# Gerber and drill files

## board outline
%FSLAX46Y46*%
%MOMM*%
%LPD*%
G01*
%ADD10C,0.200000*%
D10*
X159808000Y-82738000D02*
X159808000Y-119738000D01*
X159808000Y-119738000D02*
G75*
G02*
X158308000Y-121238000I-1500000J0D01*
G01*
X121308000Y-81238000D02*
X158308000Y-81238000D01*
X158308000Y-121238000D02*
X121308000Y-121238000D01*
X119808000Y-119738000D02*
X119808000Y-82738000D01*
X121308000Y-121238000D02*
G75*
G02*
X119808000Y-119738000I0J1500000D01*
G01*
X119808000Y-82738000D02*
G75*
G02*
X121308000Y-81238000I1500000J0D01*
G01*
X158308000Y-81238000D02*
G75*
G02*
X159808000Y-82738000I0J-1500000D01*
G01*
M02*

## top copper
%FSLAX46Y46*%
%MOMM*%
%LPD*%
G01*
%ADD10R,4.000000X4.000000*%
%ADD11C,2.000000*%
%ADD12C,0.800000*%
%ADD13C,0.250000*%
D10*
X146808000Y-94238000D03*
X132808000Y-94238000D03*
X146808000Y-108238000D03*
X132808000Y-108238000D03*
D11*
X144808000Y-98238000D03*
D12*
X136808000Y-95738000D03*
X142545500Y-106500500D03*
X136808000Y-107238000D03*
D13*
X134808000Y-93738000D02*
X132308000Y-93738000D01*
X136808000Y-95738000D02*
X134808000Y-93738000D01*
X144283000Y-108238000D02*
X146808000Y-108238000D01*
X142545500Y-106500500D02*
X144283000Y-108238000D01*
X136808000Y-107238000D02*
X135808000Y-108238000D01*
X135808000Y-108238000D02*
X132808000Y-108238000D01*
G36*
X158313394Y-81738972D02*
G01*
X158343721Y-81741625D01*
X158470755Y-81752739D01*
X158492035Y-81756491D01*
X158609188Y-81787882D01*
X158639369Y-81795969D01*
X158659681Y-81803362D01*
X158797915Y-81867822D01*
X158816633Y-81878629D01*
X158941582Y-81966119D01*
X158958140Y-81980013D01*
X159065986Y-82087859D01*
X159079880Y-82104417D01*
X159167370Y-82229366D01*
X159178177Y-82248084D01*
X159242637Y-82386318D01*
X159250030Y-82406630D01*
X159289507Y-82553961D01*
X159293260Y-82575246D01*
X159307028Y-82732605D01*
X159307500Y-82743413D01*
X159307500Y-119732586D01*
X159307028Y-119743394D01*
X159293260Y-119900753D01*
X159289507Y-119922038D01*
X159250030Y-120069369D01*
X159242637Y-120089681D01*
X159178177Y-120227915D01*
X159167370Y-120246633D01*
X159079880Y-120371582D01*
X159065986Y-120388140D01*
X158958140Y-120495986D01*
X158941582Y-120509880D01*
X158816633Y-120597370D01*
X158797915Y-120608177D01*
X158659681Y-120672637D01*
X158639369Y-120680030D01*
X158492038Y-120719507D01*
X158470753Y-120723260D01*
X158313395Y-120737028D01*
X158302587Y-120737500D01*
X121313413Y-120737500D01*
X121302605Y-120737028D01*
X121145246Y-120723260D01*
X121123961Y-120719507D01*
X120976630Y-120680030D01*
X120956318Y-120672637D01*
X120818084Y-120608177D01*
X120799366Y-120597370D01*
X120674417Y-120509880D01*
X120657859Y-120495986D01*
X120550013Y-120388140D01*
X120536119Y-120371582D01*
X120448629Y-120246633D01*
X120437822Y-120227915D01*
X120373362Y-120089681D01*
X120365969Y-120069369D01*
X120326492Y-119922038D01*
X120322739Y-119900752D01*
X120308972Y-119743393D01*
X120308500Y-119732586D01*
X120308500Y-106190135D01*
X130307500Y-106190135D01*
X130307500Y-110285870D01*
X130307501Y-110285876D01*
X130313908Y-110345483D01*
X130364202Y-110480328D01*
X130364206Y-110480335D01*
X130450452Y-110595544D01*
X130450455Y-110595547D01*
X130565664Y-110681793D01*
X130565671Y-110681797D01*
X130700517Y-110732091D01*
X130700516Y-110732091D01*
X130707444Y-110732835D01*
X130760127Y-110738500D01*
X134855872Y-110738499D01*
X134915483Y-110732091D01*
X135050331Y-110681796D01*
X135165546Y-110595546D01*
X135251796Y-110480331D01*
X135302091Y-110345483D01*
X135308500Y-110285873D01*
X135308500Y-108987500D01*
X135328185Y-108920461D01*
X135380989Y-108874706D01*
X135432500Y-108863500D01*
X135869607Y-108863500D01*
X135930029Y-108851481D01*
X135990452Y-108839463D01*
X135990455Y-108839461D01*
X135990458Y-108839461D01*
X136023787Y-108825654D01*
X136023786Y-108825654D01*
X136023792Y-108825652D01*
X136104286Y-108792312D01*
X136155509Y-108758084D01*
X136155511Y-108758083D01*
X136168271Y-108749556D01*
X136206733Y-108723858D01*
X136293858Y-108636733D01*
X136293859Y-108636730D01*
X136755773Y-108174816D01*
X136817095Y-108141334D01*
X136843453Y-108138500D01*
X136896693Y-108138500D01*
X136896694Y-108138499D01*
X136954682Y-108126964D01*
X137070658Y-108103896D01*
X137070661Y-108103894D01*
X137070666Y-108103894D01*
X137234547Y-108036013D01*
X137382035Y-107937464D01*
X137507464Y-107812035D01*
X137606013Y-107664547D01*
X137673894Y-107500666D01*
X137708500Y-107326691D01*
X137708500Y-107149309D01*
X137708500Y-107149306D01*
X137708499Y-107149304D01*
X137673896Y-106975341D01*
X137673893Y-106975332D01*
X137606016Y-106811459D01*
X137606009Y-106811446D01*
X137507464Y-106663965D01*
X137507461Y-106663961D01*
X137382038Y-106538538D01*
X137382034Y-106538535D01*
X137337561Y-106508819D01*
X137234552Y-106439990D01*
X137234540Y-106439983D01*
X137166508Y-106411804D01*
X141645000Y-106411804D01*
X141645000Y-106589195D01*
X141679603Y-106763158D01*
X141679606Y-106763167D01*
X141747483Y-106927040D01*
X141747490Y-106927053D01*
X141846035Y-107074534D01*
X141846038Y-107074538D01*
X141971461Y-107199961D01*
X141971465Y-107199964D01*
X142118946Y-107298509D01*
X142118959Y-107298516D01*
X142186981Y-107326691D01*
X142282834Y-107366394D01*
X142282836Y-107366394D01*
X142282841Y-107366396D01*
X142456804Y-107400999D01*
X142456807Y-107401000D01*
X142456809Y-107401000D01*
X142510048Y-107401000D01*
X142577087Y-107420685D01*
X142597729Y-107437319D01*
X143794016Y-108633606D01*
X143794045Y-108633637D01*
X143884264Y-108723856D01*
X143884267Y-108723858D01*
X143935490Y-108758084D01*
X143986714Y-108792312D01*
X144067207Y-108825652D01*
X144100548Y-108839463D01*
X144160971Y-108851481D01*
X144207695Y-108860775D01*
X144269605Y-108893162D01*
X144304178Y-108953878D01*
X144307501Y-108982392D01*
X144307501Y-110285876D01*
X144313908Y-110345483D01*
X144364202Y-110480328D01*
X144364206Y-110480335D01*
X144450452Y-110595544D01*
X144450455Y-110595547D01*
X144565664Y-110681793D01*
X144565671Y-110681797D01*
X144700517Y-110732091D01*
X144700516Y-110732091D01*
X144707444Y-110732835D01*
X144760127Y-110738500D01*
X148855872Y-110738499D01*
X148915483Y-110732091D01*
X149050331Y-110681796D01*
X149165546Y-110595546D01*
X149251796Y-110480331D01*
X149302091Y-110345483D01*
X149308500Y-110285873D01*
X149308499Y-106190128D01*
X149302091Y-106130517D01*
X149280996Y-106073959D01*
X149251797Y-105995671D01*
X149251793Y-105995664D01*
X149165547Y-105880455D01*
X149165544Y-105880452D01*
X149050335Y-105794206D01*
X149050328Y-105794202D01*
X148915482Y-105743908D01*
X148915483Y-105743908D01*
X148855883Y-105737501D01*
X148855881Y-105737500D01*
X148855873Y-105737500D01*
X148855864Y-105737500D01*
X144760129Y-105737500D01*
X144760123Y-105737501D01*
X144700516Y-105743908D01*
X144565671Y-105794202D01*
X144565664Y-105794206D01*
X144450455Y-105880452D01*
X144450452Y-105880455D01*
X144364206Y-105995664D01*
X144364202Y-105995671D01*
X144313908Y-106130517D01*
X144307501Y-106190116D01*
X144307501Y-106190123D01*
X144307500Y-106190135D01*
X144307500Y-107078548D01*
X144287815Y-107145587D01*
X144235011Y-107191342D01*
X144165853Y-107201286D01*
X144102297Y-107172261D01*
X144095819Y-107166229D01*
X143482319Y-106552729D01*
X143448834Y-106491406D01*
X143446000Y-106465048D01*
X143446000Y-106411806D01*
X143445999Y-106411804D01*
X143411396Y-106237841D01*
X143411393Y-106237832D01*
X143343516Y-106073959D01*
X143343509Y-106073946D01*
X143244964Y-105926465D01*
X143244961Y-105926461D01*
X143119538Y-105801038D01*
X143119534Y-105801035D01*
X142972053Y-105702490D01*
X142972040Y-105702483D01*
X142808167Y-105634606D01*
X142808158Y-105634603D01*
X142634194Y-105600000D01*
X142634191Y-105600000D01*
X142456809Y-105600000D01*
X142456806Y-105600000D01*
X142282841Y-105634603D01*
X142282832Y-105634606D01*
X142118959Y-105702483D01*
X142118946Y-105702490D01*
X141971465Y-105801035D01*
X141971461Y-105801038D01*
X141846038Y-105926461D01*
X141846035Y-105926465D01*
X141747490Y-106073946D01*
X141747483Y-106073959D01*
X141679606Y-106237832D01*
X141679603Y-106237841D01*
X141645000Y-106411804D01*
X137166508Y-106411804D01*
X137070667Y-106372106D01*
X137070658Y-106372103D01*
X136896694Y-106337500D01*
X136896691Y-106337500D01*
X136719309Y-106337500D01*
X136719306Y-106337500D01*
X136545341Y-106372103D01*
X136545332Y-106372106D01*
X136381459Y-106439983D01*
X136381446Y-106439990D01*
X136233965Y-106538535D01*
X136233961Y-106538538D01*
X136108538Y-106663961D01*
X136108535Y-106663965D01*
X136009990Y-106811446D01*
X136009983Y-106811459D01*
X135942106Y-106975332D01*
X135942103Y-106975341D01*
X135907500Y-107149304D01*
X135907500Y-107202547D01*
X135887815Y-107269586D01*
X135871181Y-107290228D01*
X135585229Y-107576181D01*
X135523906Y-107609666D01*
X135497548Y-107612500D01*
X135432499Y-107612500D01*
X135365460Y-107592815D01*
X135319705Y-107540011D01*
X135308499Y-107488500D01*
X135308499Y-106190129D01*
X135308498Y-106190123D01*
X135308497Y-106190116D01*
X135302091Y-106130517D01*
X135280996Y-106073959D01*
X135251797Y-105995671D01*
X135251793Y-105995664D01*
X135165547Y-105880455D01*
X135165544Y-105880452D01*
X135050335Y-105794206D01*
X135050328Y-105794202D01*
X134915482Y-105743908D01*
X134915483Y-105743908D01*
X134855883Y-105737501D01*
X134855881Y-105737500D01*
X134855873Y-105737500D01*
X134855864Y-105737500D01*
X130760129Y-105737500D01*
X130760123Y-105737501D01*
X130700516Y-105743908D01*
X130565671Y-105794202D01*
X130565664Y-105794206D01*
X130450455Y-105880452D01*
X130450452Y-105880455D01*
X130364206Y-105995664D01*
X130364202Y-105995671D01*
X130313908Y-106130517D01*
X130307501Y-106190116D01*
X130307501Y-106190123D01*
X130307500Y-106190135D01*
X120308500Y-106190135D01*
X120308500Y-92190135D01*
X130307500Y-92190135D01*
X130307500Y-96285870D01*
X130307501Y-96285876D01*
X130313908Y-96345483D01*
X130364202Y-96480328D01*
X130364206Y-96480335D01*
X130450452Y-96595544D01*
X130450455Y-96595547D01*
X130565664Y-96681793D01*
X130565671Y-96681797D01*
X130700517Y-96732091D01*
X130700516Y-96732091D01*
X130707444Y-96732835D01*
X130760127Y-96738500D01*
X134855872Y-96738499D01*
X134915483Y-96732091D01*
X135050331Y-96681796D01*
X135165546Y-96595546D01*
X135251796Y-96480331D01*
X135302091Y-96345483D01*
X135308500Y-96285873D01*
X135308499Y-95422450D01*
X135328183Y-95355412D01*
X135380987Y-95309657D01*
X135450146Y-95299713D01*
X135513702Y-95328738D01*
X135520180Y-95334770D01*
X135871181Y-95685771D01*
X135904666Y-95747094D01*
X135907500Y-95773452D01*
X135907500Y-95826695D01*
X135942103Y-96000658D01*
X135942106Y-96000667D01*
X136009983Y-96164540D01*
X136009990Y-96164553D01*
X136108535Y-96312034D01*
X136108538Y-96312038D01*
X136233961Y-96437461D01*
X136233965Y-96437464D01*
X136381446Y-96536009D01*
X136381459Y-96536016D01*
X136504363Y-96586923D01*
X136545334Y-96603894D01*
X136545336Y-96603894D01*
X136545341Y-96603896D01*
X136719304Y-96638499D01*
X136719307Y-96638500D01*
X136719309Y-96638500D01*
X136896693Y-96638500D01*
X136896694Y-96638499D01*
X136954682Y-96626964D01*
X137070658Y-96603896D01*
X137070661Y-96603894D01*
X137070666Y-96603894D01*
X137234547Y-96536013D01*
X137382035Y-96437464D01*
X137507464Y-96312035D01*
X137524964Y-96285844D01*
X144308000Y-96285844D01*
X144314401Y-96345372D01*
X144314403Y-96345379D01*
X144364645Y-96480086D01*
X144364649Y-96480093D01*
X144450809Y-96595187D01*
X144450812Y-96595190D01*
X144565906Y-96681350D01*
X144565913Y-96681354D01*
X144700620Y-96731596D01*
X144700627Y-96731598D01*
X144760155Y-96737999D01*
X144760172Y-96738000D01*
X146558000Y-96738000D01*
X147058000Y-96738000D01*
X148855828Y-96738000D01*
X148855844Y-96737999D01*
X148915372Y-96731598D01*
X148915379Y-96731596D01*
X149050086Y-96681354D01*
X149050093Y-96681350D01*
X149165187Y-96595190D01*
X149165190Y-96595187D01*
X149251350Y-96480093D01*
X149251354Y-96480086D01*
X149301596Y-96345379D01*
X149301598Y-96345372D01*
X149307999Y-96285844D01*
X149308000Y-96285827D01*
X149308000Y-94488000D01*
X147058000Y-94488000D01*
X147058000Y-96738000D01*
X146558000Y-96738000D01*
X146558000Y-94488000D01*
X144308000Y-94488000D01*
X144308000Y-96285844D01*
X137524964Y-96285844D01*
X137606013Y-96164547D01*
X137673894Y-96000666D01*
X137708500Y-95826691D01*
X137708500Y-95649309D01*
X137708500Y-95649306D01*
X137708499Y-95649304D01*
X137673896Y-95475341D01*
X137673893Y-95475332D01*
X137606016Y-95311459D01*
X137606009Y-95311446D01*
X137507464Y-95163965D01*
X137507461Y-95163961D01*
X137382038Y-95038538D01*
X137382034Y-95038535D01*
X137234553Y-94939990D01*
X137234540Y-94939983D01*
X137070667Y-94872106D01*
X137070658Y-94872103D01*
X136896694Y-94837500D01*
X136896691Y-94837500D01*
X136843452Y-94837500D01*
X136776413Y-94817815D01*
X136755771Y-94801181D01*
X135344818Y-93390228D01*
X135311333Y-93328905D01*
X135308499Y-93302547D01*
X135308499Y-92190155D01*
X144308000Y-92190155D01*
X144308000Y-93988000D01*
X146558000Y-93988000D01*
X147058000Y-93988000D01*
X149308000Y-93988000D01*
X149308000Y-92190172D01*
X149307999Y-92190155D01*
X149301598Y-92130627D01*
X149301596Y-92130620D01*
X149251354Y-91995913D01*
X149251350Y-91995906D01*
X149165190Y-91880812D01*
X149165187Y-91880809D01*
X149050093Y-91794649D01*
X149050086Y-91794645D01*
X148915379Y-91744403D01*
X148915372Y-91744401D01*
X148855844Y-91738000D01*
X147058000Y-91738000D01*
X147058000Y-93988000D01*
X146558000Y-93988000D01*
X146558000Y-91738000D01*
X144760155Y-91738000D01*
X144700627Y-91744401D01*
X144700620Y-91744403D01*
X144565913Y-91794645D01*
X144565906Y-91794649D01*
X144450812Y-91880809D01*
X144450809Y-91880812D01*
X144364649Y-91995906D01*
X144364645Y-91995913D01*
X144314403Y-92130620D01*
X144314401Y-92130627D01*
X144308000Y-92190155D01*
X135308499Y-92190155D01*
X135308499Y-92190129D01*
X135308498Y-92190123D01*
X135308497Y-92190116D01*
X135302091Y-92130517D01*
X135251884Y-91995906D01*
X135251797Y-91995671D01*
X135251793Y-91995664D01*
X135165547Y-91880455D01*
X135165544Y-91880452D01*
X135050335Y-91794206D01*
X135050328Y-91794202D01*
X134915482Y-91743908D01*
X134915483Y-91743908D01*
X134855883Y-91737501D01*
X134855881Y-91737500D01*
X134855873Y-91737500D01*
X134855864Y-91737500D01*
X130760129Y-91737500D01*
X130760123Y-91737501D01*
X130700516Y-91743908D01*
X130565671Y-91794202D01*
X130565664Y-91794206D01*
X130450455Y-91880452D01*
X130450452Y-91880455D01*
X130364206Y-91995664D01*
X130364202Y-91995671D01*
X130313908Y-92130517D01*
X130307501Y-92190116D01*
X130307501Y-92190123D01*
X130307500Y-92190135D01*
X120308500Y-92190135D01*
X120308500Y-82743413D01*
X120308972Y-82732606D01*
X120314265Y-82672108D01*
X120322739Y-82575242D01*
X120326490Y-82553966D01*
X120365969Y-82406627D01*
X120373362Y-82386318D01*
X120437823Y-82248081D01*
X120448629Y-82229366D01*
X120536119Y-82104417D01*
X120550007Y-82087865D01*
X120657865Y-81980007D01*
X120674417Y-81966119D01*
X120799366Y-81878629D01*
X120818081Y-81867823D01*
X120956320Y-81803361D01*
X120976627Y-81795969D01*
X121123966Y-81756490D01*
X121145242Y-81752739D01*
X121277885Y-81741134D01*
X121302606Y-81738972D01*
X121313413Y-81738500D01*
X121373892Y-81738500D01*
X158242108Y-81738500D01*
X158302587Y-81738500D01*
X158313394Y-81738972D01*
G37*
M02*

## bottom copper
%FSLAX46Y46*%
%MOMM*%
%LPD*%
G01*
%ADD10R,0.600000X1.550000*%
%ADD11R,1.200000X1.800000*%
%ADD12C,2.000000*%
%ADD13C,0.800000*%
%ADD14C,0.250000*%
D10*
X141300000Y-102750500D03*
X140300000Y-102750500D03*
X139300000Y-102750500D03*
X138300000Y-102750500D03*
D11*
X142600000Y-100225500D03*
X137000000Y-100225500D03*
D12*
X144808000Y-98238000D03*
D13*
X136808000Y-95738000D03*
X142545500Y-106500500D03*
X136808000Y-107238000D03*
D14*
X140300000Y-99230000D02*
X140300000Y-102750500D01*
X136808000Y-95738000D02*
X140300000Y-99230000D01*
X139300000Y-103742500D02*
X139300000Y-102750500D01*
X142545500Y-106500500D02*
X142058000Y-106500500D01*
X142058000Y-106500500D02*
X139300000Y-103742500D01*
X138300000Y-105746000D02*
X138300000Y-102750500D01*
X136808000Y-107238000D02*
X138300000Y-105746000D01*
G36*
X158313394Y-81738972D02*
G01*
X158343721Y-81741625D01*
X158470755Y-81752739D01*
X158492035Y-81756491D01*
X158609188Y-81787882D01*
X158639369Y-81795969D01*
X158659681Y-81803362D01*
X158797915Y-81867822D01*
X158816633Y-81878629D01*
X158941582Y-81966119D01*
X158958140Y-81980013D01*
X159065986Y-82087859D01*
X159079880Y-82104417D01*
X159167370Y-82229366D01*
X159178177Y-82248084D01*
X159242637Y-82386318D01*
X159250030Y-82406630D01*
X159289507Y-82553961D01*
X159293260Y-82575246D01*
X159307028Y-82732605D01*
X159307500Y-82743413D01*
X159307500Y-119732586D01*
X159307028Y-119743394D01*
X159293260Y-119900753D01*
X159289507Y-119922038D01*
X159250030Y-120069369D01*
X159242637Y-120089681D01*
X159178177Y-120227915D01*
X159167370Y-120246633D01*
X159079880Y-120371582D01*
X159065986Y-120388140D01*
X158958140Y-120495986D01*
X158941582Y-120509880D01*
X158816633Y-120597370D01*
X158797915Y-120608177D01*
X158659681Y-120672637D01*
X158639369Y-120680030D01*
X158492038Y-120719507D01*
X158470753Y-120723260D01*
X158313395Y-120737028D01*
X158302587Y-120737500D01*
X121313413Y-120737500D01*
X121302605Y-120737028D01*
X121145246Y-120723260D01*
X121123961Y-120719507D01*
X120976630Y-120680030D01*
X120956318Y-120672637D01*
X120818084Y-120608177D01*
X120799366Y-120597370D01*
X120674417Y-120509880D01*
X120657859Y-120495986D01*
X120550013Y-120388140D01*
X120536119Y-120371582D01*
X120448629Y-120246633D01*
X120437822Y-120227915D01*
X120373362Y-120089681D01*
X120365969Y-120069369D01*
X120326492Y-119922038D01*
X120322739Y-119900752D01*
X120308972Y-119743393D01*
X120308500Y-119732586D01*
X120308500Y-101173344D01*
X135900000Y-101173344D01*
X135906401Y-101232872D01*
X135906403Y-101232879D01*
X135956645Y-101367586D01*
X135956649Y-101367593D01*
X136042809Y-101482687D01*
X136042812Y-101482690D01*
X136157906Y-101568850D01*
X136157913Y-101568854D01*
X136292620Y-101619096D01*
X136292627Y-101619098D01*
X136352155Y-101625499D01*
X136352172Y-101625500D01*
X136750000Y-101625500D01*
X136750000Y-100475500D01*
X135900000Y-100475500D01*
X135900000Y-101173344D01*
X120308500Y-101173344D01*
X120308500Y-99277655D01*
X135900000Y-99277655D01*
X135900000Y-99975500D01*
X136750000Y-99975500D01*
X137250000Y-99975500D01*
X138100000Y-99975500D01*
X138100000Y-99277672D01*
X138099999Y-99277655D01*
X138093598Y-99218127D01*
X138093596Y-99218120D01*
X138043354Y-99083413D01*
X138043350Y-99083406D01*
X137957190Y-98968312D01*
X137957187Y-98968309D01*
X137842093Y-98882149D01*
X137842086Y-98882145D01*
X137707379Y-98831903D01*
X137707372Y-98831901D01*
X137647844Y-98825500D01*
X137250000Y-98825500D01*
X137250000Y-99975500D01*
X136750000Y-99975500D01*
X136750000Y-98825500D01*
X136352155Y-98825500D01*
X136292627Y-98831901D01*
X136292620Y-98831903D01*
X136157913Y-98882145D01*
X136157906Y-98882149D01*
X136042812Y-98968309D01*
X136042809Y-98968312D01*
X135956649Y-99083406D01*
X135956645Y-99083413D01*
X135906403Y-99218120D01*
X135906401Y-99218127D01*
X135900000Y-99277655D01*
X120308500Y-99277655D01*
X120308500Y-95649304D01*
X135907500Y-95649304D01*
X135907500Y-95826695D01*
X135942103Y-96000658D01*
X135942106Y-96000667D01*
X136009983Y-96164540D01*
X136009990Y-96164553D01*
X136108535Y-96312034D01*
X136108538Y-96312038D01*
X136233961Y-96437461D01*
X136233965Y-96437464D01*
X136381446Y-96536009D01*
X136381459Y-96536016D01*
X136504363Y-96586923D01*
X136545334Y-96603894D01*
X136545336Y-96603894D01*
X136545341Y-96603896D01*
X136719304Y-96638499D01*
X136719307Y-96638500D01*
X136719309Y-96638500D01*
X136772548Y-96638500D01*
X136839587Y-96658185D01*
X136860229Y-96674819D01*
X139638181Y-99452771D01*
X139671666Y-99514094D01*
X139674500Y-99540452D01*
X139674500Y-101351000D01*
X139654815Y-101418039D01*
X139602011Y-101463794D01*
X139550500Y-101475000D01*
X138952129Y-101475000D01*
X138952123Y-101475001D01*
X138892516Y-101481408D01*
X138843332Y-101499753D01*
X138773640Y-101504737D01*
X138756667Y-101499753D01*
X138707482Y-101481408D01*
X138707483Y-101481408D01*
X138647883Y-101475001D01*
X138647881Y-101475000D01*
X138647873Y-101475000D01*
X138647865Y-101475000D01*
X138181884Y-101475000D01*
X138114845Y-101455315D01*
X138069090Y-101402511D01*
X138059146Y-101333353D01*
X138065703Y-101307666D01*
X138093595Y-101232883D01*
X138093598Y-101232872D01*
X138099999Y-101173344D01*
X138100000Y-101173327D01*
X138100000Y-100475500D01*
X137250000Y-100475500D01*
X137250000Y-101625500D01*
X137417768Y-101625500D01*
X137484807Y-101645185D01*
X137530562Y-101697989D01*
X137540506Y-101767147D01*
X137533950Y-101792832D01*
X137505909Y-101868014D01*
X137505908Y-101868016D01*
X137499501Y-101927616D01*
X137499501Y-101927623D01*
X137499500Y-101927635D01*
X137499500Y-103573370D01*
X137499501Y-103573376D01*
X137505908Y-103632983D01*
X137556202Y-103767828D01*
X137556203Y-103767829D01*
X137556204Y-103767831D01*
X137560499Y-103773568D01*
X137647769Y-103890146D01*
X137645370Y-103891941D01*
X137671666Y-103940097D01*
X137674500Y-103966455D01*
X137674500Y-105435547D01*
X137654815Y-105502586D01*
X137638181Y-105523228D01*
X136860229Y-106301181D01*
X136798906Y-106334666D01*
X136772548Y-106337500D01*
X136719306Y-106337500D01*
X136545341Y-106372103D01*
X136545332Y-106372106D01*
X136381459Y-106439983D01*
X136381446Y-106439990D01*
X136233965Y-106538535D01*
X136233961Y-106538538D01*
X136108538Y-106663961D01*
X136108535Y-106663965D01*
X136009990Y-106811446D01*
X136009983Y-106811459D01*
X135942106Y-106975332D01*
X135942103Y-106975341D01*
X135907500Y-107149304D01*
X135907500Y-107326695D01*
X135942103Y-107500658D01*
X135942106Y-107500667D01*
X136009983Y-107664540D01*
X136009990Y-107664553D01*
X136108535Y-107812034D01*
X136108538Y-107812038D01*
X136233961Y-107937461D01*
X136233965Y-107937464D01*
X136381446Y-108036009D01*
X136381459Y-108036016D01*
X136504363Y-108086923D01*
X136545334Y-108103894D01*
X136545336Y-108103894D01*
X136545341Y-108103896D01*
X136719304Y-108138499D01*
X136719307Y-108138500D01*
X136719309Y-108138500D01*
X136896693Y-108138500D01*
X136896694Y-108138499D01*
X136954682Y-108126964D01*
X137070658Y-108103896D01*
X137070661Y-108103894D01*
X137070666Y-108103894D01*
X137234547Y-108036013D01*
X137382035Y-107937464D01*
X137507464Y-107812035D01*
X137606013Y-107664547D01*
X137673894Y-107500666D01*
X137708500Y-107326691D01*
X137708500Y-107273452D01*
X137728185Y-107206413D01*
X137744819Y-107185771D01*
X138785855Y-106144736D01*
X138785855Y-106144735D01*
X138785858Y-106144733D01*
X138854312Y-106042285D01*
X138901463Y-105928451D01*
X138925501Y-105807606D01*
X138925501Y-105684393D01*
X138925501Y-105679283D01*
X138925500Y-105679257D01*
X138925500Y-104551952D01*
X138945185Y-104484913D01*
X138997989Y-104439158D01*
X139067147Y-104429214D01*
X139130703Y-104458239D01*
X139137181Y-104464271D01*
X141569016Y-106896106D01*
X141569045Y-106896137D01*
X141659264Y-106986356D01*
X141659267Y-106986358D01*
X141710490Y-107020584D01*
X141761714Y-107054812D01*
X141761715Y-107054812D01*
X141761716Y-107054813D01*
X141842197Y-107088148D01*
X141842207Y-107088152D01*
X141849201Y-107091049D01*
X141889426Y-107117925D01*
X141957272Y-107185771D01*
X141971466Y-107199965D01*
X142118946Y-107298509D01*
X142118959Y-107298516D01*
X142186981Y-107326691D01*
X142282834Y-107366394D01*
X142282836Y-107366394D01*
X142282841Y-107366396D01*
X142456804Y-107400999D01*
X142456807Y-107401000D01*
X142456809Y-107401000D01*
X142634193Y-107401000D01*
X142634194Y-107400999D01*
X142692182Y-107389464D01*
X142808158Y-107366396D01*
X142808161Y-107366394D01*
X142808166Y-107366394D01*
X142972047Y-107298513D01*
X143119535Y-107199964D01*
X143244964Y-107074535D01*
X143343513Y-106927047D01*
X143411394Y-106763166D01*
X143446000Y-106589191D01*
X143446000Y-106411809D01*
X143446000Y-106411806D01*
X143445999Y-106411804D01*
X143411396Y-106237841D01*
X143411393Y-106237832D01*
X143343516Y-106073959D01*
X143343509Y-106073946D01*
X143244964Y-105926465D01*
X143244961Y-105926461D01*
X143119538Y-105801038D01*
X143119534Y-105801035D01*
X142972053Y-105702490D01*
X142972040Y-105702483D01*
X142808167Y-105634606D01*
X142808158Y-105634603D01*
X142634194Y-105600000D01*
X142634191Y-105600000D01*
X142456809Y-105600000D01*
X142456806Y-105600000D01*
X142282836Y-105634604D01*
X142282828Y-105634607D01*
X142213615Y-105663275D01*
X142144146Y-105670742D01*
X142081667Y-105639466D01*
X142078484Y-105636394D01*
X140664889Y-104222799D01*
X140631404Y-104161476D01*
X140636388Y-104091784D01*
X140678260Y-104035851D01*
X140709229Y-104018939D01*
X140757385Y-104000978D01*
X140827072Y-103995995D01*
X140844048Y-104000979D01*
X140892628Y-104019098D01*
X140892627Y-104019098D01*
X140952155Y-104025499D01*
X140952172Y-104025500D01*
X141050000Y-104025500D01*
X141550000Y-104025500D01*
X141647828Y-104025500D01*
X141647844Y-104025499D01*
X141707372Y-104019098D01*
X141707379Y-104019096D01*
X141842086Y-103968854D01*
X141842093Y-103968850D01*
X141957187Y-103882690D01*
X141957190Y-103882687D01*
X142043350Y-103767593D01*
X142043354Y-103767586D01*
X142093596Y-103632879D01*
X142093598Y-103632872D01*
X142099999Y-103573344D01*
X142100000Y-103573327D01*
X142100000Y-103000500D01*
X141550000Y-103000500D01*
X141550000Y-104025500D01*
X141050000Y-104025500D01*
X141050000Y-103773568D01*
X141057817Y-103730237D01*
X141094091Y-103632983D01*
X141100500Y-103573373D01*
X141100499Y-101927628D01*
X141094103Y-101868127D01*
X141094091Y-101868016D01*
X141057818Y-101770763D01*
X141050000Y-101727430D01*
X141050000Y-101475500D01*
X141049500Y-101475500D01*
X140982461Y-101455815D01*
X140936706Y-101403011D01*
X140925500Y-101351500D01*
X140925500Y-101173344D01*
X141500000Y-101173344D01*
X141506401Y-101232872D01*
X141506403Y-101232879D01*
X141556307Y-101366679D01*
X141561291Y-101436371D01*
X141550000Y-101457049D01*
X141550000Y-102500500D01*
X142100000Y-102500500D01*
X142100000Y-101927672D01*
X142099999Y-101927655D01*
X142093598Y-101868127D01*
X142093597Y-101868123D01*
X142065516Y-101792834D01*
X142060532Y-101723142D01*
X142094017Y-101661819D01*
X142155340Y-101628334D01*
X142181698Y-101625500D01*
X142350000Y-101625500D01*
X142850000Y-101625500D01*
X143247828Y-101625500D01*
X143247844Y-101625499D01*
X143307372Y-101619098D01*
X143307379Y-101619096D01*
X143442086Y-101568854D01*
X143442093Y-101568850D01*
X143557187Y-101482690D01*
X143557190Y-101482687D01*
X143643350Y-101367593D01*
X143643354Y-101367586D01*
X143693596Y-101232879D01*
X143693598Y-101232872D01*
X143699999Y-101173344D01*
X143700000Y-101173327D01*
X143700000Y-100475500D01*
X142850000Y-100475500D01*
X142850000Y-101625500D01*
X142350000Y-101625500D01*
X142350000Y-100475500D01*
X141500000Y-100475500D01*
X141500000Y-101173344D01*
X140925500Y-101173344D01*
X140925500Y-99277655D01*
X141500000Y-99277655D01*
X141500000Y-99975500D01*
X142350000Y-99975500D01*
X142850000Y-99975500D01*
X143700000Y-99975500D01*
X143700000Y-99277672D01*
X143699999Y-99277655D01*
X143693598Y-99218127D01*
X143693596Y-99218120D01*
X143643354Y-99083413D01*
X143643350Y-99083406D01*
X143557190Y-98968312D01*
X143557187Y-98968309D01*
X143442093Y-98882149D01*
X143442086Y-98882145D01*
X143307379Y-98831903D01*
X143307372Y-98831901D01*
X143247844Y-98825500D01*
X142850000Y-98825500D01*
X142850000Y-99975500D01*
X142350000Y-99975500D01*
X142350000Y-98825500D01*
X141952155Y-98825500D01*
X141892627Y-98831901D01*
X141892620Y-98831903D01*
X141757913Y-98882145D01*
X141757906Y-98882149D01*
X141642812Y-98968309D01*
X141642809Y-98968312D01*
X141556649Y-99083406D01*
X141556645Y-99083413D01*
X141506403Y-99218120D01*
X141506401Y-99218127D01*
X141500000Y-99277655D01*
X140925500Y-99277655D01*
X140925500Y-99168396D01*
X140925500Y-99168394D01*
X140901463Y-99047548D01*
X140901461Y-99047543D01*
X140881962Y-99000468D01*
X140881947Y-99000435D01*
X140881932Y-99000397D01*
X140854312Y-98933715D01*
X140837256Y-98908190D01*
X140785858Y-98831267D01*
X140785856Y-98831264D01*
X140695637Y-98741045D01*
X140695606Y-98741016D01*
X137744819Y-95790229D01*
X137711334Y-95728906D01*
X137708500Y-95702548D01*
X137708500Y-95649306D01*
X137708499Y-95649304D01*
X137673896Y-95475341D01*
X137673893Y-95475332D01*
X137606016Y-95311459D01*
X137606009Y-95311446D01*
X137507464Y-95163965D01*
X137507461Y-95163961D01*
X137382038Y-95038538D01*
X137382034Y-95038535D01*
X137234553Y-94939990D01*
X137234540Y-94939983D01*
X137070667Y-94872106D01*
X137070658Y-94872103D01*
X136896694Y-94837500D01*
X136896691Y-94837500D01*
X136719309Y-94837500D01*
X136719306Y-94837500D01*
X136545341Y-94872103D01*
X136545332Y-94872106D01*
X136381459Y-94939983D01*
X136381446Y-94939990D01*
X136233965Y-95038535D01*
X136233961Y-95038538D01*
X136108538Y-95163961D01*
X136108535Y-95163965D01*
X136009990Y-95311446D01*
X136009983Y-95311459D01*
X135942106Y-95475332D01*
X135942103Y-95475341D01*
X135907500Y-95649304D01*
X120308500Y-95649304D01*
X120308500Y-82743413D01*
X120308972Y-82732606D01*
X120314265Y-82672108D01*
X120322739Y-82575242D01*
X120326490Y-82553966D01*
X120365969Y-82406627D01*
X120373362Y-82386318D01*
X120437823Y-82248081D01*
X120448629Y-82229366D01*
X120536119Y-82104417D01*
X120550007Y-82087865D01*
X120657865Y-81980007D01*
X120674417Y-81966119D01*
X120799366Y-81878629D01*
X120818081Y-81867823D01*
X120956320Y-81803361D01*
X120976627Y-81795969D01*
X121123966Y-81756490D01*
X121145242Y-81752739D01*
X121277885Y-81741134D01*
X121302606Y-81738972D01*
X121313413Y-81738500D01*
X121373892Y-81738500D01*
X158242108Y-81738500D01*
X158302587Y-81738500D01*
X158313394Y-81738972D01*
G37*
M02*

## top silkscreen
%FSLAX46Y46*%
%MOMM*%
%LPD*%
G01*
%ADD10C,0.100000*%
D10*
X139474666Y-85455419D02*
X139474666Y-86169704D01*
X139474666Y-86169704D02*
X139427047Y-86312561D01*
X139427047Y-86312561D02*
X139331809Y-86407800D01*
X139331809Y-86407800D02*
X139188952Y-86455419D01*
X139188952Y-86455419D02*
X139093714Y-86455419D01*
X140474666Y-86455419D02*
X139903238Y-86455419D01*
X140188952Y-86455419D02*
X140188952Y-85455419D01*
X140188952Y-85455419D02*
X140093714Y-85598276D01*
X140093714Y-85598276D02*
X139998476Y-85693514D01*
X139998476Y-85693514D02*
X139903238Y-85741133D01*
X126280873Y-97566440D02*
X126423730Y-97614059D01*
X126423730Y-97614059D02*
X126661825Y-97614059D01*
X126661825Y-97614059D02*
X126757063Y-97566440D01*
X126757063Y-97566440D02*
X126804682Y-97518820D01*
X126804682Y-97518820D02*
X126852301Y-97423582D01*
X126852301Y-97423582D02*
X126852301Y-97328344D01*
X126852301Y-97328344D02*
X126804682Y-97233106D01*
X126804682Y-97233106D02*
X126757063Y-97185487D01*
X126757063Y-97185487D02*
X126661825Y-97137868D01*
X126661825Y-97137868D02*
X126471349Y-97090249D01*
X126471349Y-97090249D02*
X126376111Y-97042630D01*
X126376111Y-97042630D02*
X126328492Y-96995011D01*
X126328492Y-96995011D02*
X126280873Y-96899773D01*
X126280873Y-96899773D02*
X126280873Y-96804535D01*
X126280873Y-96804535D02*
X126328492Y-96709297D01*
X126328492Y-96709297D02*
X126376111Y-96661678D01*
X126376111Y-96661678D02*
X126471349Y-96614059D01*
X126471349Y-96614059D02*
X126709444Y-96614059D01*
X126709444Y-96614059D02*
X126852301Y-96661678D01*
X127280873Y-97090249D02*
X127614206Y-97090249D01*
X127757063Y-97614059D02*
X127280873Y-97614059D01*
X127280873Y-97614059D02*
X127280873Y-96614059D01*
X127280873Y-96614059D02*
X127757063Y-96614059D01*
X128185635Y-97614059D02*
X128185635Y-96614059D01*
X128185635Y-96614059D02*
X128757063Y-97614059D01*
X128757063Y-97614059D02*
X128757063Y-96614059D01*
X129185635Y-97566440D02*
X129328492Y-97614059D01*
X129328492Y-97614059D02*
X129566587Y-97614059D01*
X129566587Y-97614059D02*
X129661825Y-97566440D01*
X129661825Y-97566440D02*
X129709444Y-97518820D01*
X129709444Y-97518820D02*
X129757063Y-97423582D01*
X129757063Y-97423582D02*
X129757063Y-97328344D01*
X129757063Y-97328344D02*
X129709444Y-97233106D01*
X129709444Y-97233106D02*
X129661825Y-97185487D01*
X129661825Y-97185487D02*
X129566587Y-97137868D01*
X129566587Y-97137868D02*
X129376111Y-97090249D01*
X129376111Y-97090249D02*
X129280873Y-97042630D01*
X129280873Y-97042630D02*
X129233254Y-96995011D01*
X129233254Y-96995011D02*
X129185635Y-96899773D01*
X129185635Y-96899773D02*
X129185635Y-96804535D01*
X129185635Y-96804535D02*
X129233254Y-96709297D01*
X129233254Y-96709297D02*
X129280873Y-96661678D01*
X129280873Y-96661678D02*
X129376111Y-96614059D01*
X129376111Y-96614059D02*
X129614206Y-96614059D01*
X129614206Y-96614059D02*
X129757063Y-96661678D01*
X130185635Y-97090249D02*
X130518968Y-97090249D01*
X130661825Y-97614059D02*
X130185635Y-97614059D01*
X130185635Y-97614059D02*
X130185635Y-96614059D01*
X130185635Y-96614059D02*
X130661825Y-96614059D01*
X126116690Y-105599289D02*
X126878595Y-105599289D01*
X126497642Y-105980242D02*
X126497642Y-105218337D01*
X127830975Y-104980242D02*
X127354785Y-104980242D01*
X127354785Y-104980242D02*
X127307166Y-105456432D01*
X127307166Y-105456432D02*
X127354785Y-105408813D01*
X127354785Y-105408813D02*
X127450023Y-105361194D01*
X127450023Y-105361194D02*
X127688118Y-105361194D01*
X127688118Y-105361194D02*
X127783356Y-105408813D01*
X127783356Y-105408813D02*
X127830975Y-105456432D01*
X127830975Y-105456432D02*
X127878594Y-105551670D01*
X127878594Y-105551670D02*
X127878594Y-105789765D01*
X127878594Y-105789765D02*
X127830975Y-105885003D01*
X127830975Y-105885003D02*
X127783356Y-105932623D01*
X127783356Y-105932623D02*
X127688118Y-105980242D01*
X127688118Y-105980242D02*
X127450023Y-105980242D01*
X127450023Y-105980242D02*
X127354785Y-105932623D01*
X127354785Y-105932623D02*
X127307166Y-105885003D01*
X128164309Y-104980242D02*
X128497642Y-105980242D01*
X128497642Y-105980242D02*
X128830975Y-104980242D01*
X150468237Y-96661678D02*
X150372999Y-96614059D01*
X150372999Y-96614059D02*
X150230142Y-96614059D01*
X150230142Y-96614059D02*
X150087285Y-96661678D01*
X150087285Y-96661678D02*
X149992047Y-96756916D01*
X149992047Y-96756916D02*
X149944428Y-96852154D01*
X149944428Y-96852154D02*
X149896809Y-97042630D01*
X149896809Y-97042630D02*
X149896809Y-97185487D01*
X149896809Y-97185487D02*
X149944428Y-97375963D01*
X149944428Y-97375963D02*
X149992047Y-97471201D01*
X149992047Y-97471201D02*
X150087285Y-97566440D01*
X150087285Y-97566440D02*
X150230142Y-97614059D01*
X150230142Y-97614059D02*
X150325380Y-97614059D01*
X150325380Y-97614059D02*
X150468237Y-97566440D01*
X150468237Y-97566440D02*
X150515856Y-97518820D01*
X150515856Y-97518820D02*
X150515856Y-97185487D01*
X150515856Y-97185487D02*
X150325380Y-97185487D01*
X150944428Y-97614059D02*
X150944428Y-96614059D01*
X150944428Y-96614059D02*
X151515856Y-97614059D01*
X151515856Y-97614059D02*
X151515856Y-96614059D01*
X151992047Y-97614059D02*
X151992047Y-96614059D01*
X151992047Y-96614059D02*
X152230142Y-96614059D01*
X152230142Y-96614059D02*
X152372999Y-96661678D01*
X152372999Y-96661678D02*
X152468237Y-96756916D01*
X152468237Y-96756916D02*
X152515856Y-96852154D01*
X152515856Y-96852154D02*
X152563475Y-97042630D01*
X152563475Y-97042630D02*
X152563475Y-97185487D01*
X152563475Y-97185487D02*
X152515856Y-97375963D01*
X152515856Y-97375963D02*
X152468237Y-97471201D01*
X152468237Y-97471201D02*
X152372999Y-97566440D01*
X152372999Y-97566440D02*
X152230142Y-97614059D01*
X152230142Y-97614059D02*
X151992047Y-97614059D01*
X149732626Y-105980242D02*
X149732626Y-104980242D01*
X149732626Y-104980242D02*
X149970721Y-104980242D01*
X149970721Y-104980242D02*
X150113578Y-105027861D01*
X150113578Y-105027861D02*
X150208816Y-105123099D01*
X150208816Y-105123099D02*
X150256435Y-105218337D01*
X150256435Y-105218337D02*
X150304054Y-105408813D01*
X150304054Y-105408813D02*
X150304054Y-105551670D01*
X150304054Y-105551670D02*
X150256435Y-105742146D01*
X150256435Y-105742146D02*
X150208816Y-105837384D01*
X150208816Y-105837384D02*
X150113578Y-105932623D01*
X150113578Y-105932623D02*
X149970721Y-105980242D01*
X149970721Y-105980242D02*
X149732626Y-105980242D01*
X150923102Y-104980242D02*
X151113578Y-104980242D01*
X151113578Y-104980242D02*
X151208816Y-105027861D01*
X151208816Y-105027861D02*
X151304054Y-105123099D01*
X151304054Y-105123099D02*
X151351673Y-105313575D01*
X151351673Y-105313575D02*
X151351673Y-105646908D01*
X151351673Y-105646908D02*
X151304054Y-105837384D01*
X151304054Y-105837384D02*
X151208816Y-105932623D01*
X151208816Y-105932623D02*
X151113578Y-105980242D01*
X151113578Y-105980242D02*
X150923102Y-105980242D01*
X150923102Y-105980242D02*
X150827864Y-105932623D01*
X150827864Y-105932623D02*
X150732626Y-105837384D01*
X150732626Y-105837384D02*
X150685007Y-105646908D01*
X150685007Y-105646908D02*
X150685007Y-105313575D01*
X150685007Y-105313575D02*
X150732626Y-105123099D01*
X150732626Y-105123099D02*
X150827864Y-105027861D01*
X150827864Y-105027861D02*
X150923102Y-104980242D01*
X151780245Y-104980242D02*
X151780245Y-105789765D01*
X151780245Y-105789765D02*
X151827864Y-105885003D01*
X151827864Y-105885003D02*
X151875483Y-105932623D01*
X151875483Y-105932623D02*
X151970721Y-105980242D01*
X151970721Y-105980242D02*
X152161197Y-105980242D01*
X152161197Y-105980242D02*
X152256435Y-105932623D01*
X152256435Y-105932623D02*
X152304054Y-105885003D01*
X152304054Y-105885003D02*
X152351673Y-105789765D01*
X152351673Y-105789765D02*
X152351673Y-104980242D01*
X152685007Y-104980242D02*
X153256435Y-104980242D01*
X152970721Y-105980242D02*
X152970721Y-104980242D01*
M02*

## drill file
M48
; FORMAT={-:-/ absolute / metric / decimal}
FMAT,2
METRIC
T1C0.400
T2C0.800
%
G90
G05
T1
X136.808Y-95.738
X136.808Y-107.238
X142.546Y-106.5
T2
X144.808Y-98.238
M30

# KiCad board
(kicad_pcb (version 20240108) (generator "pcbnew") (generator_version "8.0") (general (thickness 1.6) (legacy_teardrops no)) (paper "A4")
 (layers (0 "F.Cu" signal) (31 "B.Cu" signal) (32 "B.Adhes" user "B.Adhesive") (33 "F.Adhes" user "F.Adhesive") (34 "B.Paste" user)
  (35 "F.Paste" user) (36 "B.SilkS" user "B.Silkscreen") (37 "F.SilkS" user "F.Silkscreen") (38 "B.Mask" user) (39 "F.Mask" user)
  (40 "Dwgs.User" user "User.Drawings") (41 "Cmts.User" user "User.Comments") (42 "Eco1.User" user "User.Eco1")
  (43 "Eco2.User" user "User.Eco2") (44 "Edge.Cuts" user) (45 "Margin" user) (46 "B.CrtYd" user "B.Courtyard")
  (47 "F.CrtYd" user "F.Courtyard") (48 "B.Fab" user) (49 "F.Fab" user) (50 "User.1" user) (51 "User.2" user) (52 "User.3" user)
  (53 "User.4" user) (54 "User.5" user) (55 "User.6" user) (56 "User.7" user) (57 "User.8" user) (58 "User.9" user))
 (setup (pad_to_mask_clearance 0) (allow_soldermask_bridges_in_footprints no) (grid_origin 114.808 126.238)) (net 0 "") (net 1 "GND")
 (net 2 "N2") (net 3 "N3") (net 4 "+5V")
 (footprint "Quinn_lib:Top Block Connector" (layer "F.Cu") (at 139.808 101.238)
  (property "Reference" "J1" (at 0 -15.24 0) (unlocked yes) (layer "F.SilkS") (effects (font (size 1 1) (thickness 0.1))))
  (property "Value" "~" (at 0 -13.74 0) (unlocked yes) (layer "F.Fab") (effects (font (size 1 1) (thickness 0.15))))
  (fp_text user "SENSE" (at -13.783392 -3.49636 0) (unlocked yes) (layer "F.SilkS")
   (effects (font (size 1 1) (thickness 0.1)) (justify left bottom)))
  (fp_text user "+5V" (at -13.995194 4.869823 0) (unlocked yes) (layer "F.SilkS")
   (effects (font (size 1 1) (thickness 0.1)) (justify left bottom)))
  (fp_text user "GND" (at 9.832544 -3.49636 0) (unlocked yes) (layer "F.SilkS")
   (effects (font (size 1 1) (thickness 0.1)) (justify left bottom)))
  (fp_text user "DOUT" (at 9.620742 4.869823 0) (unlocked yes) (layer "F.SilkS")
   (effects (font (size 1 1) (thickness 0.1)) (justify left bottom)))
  (pad "1" smd rect (at 7 -7) (size 4 4) (layers "F.Cu" "F.Paste" "F.Mask") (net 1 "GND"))
  (pad "2" smd rect (at -7 -7) (size 4 4) (layers "F.Cu" "F.Paste" "F.Mask") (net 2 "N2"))
  (pad "3" smd rect (at 7 7) (size 4 4) (layers "F.Cu" "F.Paste" "F.Mask") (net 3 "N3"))
  (pad "4" smd rect (at -7 7) (size 4 4) (layers "F.Cu" "F.Paste" "F.Mask") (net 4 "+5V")))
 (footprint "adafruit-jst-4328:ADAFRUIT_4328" (layer "B.Cu") (at 139.8 100.9755 180)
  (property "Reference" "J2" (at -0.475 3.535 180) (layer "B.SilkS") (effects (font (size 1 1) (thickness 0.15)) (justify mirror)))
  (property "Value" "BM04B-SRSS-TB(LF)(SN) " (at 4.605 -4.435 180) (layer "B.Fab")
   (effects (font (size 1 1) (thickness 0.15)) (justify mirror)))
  (pad "1" smd rect (at -1.5 -1.775 180) (size 0.6 1.55) (layers "B.Cu" "B.Paste" "B.Mask") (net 1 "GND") (solder_mask_margin 0.102))
  (pad "2" smd rect (at -0.5 -1.775 180) (size 0.6 1.55) (layers "B.Cu" "B.Paste" "B.Mask") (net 2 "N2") (solder_mask_margin 0.102))
  (pad "3" smd rect (at 0.5 -1.775 180) (size 0.6 1.55) (layers "B.Cu" "B.Paste" "B.Mask") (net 3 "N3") (solder_mask_margin 0.102))
  (pad "4" smd rect (at 1.5 -1.775 180) (size 0.6 1.55) (layers "B.Cu" "B.Paste" "B.Mask") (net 4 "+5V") (solder_mask_margin 0.102))
  (pad "SH1" smd rect (at -2.8 0.75 180) (size 1.2 1.8) (layers "B.Cu" "B.Paste" "B.Mask") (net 1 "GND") (solder_mask_margin 0.102))
  (pad "SH2" smd rect (at 2.8 0.75 180) (size 1.2 1.8) (layers "B.Cu" "B.Paste" "B.Mask") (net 1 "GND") (solder_mask_margin 0.102)))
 (gr_line (start 159.808 82.738) (end 159.808 119.738) (stroke (width 0.2) (type default)) (layer "Edge.Cuts"))
 (gr_arc (start 159.808 119.738) (mid 159.36866 120.79866) (end 158.308 121.238) (stroke (width 0.2) (type default)) (layer "Edge.Cuts"))
 (gr_line (start 121.308 81.238) (end 158.308 81.238) (stroke (width 0.2) (type default)) (layer "Edge.Cuts"))
 (gr_line (start 158.308 121.238) (end 121.308 121.238) (stroke (width 0.2) (type default)) (layer "Edge.Cuts"))
 (gr_line (start 119.808 119.738) (end 119.808 82.738) (stroke (width 0.2) (type default)) (layer "Edge.Cuts"))
 (gr_arc (start 121.308 121.238) (mid 120.24734 120.79866) (end 119.808 119.738) (stroke (width 0.2) (type default)) (layer "Edge.Cuts"))
 (gr_arc (start 119.808 82.738) (mid 120.24734 81.67734) (end 121.308 81.238) (stroke (width 0.2) (type default)) (layer "Edge.Cuts"))
 (gr_arc (start 158.308 81.238) (mid 159.36866 81.67734) (end 159.808 82.738) (stroke (width 0.2) (type default)) (layer "Edge.Cuts"))
 (via (at 144.808 98.238) (size 2) (drill 0.8) (layers "F.Cu" "B.Cu") (free yes) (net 1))
 (segment (start 134.808 93.738) (end 132.308 93.738) (width 0.25) (layer "F.Cu") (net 2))
 (segment (start 136.808 95.738) (end 134.808 93.738) (width 0.25) (layer "F.Cu") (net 2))
 (via (at 136.808 95.738) (size 0.8) (drill 0.4) (layers "F.Cu" "B.Cu") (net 2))
 (segment (start 140.3 99.23) (end 140.3 102.7505) (width 0.25) (layer "B.Cu") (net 2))
 (segment (start 136.808 95.738) (end 140.3 99.23) (width 0.25) (layer "B.Cu") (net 2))
 (segment (start 144.283 108.238) (end 146.808 108.238) (width 0.25) (layer "F.Cu") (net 3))
 (segment (start 142.5455 106.5005) (end 144.283 108.238) (width 0.25) (layer "F.Cu") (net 3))
 (via (at 142.5455 106.5005) (size 0.8) (drill 0.4) (layers "F.Cu" "B.Cu") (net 3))
 (segment (start 139.3 103.7425) (end 139.3 102.7505) (width 0.25) (layer "B.Cu") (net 3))
 (segment (start 142.5455 106.5005) (end 142.058 106.5005) (width 0.25) (layer "B.Cu") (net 3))
 (segment (start 142.058 106.5005) (end 139.3 103.7425) (width 0.25) (layer "B.Cu") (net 3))
 (segment (start 136.808 107.238) (end 135.808 108.238) (width 0.25) (layer "F.Cu") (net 4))
 (segment (start 135.808 108.238) (end 132.808 108.238) (width 0.25) (layer "F.Cu") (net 4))
 (via (at 136.808 107.238) (size 0.8) (drill 0.4) (layers "F.Cu" "B.Cu") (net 4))
 (segment (start 138.3 105.746) (end 138.3 102.7505) (width 0.25) (layer "B.Cu") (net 4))
 (segment (start 136.808 107.238) (end 138.3 105.746) (width 0.25) (layer "B.Cu") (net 4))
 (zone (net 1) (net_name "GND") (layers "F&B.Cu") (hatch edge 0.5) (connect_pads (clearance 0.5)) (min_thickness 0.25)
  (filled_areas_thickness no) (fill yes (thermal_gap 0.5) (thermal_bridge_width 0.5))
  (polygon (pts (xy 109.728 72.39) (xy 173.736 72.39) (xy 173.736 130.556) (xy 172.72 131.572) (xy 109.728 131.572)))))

